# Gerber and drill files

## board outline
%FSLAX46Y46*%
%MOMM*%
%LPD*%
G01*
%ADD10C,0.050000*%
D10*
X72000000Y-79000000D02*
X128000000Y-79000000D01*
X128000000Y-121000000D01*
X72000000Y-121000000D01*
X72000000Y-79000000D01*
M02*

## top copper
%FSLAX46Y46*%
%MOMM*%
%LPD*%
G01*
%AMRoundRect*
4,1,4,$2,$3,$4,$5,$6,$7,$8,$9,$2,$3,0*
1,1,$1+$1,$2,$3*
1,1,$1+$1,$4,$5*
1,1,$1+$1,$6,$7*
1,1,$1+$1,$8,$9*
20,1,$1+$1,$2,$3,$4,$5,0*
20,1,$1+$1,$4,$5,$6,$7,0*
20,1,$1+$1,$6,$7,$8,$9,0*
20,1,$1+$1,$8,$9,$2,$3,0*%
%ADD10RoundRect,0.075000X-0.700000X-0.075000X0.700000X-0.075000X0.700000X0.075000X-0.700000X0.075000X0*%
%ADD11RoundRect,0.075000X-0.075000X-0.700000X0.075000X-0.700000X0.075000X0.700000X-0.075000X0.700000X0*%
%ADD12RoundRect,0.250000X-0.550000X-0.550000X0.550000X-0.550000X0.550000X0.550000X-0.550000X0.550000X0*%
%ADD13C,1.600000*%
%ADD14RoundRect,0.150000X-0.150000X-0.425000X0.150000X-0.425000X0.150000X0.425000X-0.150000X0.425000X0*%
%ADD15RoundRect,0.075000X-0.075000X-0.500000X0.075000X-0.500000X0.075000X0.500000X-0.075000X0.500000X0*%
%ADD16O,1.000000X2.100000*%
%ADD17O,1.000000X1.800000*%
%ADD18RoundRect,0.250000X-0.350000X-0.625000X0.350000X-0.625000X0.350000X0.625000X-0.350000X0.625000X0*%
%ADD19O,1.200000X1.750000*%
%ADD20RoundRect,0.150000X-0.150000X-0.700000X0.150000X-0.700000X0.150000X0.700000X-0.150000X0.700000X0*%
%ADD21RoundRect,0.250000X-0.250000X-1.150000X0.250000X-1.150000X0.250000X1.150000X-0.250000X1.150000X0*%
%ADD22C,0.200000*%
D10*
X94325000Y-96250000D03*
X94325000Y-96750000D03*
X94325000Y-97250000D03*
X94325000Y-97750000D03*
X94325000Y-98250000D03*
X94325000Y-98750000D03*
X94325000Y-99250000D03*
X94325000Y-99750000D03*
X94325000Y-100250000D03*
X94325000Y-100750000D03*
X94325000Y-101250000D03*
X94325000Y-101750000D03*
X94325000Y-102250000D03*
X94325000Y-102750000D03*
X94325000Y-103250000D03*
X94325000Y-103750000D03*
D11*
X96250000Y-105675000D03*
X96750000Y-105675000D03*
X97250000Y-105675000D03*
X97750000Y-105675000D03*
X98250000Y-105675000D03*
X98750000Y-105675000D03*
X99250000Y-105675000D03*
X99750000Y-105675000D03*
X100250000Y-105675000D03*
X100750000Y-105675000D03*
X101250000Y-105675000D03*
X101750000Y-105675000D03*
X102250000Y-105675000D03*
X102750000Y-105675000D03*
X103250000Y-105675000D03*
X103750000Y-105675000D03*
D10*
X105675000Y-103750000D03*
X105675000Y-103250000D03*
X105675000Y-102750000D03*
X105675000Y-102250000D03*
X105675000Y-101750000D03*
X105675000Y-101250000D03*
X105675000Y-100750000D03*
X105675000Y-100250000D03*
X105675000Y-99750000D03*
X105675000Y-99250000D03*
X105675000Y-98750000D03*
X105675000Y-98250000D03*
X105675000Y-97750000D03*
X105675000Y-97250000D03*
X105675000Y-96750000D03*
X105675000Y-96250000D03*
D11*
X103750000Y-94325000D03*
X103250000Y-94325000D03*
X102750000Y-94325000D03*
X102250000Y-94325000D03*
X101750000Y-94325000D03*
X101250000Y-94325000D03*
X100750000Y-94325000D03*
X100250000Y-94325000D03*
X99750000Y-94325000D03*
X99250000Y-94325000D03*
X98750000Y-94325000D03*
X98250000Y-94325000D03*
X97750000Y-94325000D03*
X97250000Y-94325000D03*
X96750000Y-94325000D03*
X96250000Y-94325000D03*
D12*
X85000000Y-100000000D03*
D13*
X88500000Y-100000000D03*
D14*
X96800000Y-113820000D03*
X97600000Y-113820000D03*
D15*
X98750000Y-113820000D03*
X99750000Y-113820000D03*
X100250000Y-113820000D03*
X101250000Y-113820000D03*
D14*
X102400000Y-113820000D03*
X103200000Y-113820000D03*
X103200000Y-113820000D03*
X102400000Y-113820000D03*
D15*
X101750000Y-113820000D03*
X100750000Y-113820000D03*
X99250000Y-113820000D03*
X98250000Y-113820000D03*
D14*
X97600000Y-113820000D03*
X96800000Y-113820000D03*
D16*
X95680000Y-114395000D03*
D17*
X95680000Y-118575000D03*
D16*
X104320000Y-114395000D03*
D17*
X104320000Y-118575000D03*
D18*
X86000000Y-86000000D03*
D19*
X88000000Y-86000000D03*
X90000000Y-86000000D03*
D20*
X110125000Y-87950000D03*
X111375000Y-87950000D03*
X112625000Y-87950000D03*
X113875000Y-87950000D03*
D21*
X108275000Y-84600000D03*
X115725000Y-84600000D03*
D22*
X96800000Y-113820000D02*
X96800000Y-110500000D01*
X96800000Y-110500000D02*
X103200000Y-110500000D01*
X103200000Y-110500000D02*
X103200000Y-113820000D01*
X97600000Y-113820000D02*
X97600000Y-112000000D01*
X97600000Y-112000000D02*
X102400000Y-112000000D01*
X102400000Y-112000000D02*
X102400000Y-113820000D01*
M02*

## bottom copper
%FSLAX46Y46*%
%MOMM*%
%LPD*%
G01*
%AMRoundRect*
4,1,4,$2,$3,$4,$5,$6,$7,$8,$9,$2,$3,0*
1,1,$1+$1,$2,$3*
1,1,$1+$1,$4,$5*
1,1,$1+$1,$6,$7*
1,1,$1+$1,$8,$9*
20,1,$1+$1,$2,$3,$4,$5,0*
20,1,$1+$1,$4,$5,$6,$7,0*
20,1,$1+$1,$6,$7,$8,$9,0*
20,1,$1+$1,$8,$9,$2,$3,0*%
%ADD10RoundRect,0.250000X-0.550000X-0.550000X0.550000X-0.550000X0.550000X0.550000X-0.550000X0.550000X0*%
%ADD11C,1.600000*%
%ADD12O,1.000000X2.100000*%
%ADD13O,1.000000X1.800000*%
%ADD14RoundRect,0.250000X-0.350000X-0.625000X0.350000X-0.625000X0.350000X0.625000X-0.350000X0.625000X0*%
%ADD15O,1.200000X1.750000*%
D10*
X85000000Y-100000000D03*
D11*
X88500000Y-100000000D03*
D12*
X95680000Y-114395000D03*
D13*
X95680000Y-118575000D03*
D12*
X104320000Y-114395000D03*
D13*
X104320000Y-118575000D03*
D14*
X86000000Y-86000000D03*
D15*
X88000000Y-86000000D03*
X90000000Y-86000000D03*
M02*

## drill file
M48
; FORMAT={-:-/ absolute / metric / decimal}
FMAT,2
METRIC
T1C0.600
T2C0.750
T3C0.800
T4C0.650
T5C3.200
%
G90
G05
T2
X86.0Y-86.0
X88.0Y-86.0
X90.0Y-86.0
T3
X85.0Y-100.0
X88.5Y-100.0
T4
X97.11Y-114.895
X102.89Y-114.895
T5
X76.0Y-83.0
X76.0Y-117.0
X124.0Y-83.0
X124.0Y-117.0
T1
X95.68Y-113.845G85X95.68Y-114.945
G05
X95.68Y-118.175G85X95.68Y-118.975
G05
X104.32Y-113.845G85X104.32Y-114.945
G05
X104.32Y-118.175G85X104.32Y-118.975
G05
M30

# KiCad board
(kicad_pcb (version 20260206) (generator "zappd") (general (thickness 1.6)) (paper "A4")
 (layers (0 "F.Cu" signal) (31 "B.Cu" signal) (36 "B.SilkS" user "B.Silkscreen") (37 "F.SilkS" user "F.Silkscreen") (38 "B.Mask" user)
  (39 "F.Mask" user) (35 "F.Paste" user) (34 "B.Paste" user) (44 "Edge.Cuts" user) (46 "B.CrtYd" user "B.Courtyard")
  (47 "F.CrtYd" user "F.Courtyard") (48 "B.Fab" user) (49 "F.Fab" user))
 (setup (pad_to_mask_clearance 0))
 (gr_rect (start 72.0 79.0) (end 128.0 121.0) (stroke (width 0.05) (type default)) (fill none) (layer "Edge.Cuts"))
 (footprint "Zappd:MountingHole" (layer "F.Cu") (at 76.0 83.0)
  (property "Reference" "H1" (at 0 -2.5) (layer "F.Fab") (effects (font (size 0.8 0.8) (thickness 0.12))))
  (pad "" np_thru_hole circle (at 0 0) (size 3.2 3.2) (drill 3.2) (layers "*.Cu" "*.Mask")))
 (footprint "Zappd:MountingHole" (layer "F.Cu") (at 124.0 83.0)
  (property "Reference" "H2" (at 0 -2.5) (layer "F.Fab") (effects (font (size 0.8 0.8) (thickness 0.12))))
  (pad "" np_thru_hole circle (at 0 0) (size 3.2 3.2) (drill 3.2) (layers "*.Cu" "*.Mask")))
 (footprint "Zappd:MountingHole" (layer "F.Cu") (at 124.0 117.0)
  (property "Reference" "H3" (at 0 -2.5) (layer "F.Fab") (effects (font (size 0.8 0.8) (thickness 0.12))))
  (pad "" np_thru_hole circle (at 0 0) (size 3.2 3.2) (drill 3.2) (layers "*.Cu" "*.Mask")))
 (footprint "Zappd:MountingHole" (layer "F.Cu") (at 76.0 117.0)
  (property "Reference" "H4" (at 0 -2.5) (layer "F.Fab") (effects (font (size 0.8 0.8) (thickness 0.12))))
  (pad "" np_thru_hole circle (at 0 0) (size 3.2 3.2) (drill 3.2) (layers "*.Cu" "*.Mask")))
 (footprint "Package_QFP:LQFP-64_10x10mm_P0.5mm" (layer "F.Cu") (at 100 100)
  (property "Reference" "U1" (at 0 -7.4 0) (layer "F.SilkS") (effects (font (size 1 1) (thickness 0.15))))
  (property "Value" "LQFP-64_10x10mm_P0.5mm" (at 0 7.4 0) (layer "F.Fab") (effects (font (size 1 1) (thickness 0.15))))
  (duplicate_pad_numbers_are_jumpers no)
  (pad "1" smd roundrect (at -5.675 -3.75) (size 1.55 0.3) (layers "F.Cu" "F.Mask" "F.Paste") (roundrect_rratio 0.25))
  (pad "2" smd roundrect (at -5.675 -3.25) (size 1.55 0.3) (layers "F.Cu" "F.Mask" "F.Paste") (roundrect_rratio 0.25))
  (pad "3" smd roundrect (at -5.675 -2.75) (size 1.55 0.3) (layers "F.Cu" "F.Mask" "F.Paste") (roundrect_rratio 0.25))
  (pad "4" smd roundrect (at -5.675 -2.25) (size 1.55 0.3) (layers "F.Cu" "F.Mask" "F.Paste") (roundrect_rratio 0.25))
  (pad "5" smd roundrect (at -5.675 -1.75) (size 1.55 0.3) (layers "F.Cu" "F.Mask" "F.Paste") (roundrect_rratio 0.25))
  (pad "6" smd roundrect (at -5.675 -1.25) (size 1.55 0.3) (layers "F.Cu" "F.Mask" "F.Paste") (roundrect_rratio 0.25))
  (pad "7" smd roundrect (at -5.675 -0.75) (size 1.55 0.3) (layers "F.Cu" "F.Mask" "F.Paste") (roundrect_rratio 0.25))
  (pad "8" smd roundrect (at -5.675 -0.25) (size 1.55 0.3) (layers "F.Cu" "F.Mask" "F.Paste") (roundrect_rratio 0.25))
  (pad "9" smd roundrect (at -5.675 0.25) (size 1.55 0.3) (layers "F.Cu" "F.Mask" "F.Paste") (roundrect_rratio 0.25))
  (pad "10" smd roundrect (at -5.675 0.75) (size 1.55 0.3) (layers "F.Cu" "F.Mask" "F.Paste") (roundrect_rratio 0.25))
  (pad "11" smd roundrect (at -5.675 1.25) (size 1.55 0.3) (layers "F.Cu" "F.Mask" "F.Paste") (roundrect_rratio 0.25))
  (pad "12" smd roundrect (at -5.675 1.75) (size 1.55 0.3) (layers "F.Cu" "F.Mask" "F.Paste") (roundrect_rratio 0.25))
  (pad "13" smd roundrect (at -5.675 2.25) (size 1.55 0.3) (layers "F.Cu" "F.Mask" "F.Paste") (roundrect_rratio 0.25))
  (pad "14" smd roundrect (at -5.675 2.75) (size 1.55 0.3) (layers "F.Cu" "F.Mask" "F.Paste") (roundrect_rratio 0.25))
  (pad "15" smd roundrect (at -5.675 3.25) (size 1.55 0.3) (layers "F.Cu" "F.Mask" "F.Paste") (roundrect_rratio 0.25))
  (pad "16" smd roundrect (at -5.675 3.75) (size 1.55 0.3) (layers "F.Cu" "F.Mask" "F.Paste") (roundrect_rratio 0.25))
  (pad "17" smd roundrect (at -3.75 5.675) (size 0.3 1.55) (layers "F.Cu" "F.Mask" "F.Paste") (roundrect_rratio 0.25))
  (pad "18" smd roundrect (at -3.25 5.675) (size 0.3 1.55) (layers "F.Cu" "F.Mask" "F.Paste") (roundrect_rratio 0.25))
  (pad "19" smd roundrect (at -2.75 5.675) (size 0.3 1.55) (layers "F.Cu" "F.Mask" "F.Paste") (roundrect_rratio 0.25))
  (pad "20" smd roundrect (at -2.25 5.675) (size 0.3 1.55) (layers "F.Cu" "F.Mask" "F.Paste") (roundrect_rratio 0.25))
  (pad "21" smd roundrect (at -1.75 5.675) (size 0.3 1.55) (layers "F.Cu" "F.Mask" "F.Paste") (roundrect_rratio 0.25))
  (pad "22" smd roundrect (at -1.25 5.675) (size 0.3 1.55) (layers "F.Cu" "F.Mask" "F.Paste") (roundrect_rratio 0.25))
  (pad "23" smd roundrect (at -0.75 5.675) (size 0.3 1.55) (layers "F.Cu" "F.Mask" "F.Paste") (roundrect_rratio 0.25))
  (pad "24" smd roundrect (at -0.25 5.675) (size 0.3 1.55) (layers "F.Cu" "F.Mask" "F.Paste") (roundrect_rratio 0.25))
  (pad "25" smd roundrect (at 0.25 5.675) (size 0.3 1.55) (layers "F.Cu" "F.Mask" "F.Paste") (roundrect_rratio 0.25))
  (pad "26" smd roundrect (at 0.75 5.675) (size 0.3 1.55) (layers "F.Cu" "F.Mask" "F.Paste") (roundrect_rratio 0.25))
  (pad "27" smd roundrect (at 1.25 5.675) (size 0.3 1.55) (layers "F.Cu" "F.Mask" "F.Paste") (roundrect_rratio 0.25))
  (pad "28" smd roundrect (at 1.75 5.675) (size 0.3 1.55) (layers "F.Cu" "F.Mask" "F.Paste") (roundrect_rratio 0.25))
  (pad "29" smd roundrect (at 2.25 5.675) (size 0.3 1.55) (layers "F.Cu" "F.Mask" "F.Paste") (roundrect_rratio 0.25))
  (pad "30" smd roundrect (at 2.75 5.675) (size 0.3 1.55) (layers "F.Cu" "F.Mask" "F.Paste") (roundrect_rratio 0.25))
  (pad "31" smd roundrect (at 3.25 5.675) (size 0.3 1.55) (layers "F.Cu" "F.Mask" "F.Paste") (roundrect_rratio 0.25))
  (pad "32" smd roundrect (at 3.75 5.675) (size 0.3 1.55) (layers "F.Cu" "F.Mask" "F.Paste") (roundrect_rratio 0.25))
  (pad "33" smd roundrect (at 5.675 3.75) (size 1.55 0.3) (layers "F.Cu" "F.Mask" "F.Paste") (roundrect_rratio 0.25))
  (pad "34" smd roundrect (at 5.675 3.25) (size 1.55 0.3) (layers "F.Cu" "F.Mask" "F.Paste") (roundrect_rratio 0.25))
  (pad "35" smd roundrect (at 5.675 2.75) (size 1.55 0.3) (layers "F.Cu" "F.Mask" "F.Paste") (roundrect_rratio 0.25))
  (pad "36" smd roundrect (at 5.675 2.25) (size 1.55 0.3) (layers "F.Cu" "F.Mask" "F.Paste") (roundrect_rratio 0.25))
  (pad "37" smd roundrect (at 5.675 1.75) (size 1.55 0.3) (layers "F.Cu" "F.Mask" "F.Paste") (roundrect_rratio 0.25))
  (pad "38" smd roundrect (at 5.675 1.25) (size 1.55 0.3) (layers "F.Cu" "F.Mask" "F.Paste") (roundrect_rratio 0.25))
  (pad "39" smd roundrect (at 5.675 0.75) (size 1.55 0.3) (layers "F.Cu" "F.Mask" "F.Paste") (roundrect_rratio 0.25))
  (pad "40" smd roundrect (at 5.675 0.25) (size 1.55 0.3) (layers "F.Cu" "F.Mask" "F.Paste") (roundrect_rratio 0.25))
  (pad "41" smd roundrect (at 5.675 -0.25) (size 1.55 0.3) (layers "F.Cu" "F.Mask" "F.Paste") (roundrect_rratio 0.25))
  (pad "42" smd roundrect (at 5.675 -0.75) (size 1.55 0.3) (layers "F.Cu" "F.Mask" "F.Paste") (roundrect_rratio 0.25))
  (pad "43" smd roundrect (at 5.675 -1.25) (size 1.55 0.3) (layers "F.Cu" "F.Mask" "F.Paste") (roundrect_rratio 0.25))
  (pad "44" smd roundrect (at 5.675 -1.75) (size 1.55 0.3) (layers "F.Cu" "F.Mask" "F.Paste") (roundrect_rratio 0.25))
  (pad "45" smd roundrect (at 5.675 -2.25) (size 1.55 0.3) (layers "F.Cu" "F.Mask" "F.Paste") (roundrect_rratio 0.25))
  (pad "46" smd roundrect (at 5.675 -2.75) (size 1.55 0.3) (layers "F.Cu" "F.Mask" "F.Paste") (roundrect_rratio 0.25))
  (pad "47" smd roundrect (at 5.675 -3.25) (size 1.55 0.3) (layers "F.Cu" "F.Mask" "F.Paste") (roundrect_rratio 0.25))
  (pad "48" smd roundrect (at 5.675 -3.75) (size 1.55 0.3) (layers "F.Cu" "F.Mask" "F.Paste") (roundrect_rratio 0.25))
  (pad "49" smd roundrect (at 3.75 -5.675) (size 0.3 1.55) (layers "F.Cu" "F.Mask" "F.Paste") (roundrect_rratio 0.25))
  (pad "50" smd roundrect (at 3.25 -5.675) (size 0.3 1.55) (layers "F.Cu" "F.Mask" "F.Paste") (roundrect_rratio 0.25))
  (pad "51" smd roundrect (at 2.75 -5.675) (size 0.3 1.55) (layers "F.Cu" "F.Mask" "F.Paste") (roundrect_rratio 0.25))
  (pad "52" smd roundrect (at 2.25 -5.675) (size 0.3 1.55) (layers "F.Cu" "F.Mask" "F.Paste") (roundrect_rratio 0.25))
  (pad "53" smd roundrect (at 1.75 -5.675) (size 0.3 1.55) (layers "F.Cu" "F.Mask" "F.Paste") (roundrect_rratio 0.25))
  (pad "54" smd roundrect (at 1.25 -5.675) (size 0.3 1.55) (layers "F.Cu" "F.Mask" "F.Paste") (roundrect_rratio 0.25))
  (pad "55" smd roundrect (at 0.75 -5.675) (size 0.3 1.55) (layers "F.Cu" "F.Mask" "F.Paste") (roundrect_rratio 0.25))
  (pad "56" smd roundrect (at 0.25 -5.675) (size 0.3 1.55) (layers "F.Cu" "F.Mask" "F.Paste") (roundrect_rratio 0.25))
  (pad "57" smd roundrect (at -0.25 -5.675) (size 0.3 1.55) (layers "F.Cu" "F.Mask" "F.Paste") (roundrect_rratio 0.25))
  (pad "58" smd roundrect (at -0.75 -5.675) (size 0.3 1.55) (layers "F.Cu" "F.Mask" "F.Paste") (roundrect_rratio 0.25))
  (pad "59" smd roundrect (at -1.25 -5.675) (size 0.3 1.55) (layers "F.Cu" "F.Mask" "F.Paste") (roundrect_rratio 0.25))
  (pad "60" smd roundrect (at -1.75 -5.675) (size 0.3 1.55) (layers "F.Cu" "F.Mask" "F.Paste") (roundrect_rratio 0.25))
  (pad "61" smd roundrect (at -2.25 -5.675) (size 0.3 1.55) (layers "F.Cu" "F.Mask" "F.Paste") (roundrect_rratio 0.25))
  (pad "62" smd roundrect (at -2.75 -5.675) (size 0.3 1.55) (layers "F.Cu" "F.Mask" "F.Paste") (roundrect_rratio 0.25))
  (pad "63" smd roundrect (at -3.25 -5.675) (size 0.3 1.55) (layers "F.Cu" "F.Mask" "F.Paste") (roundrect_rratio 0.25))
  (pad "64" smd roundrect (at -3.75 -5.675) (size 0.3 1.55) (layers "F.Cu" "F.Mask" "F.Paste") (roundrect_rratio 0.25)))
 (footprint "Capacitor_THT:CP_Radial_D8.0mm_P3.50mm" (layer "F.Cu") (at 85 100)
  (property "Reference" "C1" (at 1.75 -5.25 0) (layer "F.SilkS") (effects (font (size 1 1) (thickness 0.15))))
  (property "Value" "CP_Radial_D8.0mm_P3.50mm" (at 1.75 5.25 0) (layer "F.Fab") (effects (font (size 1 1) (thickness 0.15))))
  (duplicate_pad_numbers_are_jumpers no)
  (pad "1" thru_hole roundrect (at 0 0) (size 1.6 1.6) (drill 0.8) (layers "*.Cu" "*.Mask") (remove_unused_layers no)
   (roundrect_rratio 0.15625))
  (pad "2" thru_hole circle (at 3.5 0) (size 1.6 1.6) (drill 0.8) (layers "*.Cu" "*.Mask") (remove_unused_layers no)))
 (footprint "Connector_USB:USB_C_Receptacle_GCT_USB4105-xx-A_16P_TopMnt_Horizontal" (layer "F.Cu") (at 100 117.5)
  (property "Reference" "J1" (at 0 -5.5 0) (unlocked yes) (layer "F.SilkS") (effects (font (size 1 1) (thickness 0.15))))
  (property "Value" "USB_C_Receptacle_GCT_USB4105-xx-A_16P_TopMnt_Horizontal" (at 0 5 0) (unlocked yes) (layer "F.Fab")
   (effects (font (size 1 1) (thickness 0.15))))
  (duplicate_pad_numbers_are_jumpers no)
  (pad "" np_thru_hole circle (at -2.89 -2.605) (size 0.65 0.65) (drill 0.65) (layers "*.Cu" "*.Mask"))
  (pad "" np_thru_hole circle (at 2.89 -2.605) (size 0.65 0.65) (drill 0.65) (layers "*.Cu" "*.Mask"))
  (pad "A1" smd roundrect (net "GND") (at -3.2 -3.68) (size 0.6 1.15) (layers "F.Cu" "F.Mask" "F.Paste") (roundrect_rratio 0.25))
  (pad "A4" smd roundrect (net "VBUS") (at -2.4 -3.68) (size 0.6 1.15) (layers "F.Cu" "F.Mask" "F.Paste") (roundrect_rratio 0.25))
  (pad "A5" smd roundrect (at -1.25 -3.68) (size 0.3 1.15) (layers "F.Cu" "F.Mask" "F.Paste") (roundrect_rratio 0.25))
  (pad "A6" smd roundrect (at -0.25 -3.68) (size 0.3 1.15) (layers "F.Cu" "F.Mask" "F.Paste") (roundrect_rratio 0.25))
  (pad "A7" smd roundrect (at 0.25 -3.68) (size 0.3 1.15) (layers "F.Cu" "F.Mask" "F.Paste") (roundrect_rratio 0.25))
  (pad "A8" smd roundrect (at 1.25 -3.68) (size 0.3 1.15) (layers "F.Cu" "F.Mask" "F.Paste") (roundrect_rratio 0.25))
  (pad "A9" smd roundrect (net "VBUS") (at 2.4 -3.68) (size 0.6 1.15) (layers "F.Cu" "F.Mask" "F.Paste") (roundrect_rratio 0.25))
  (pad "A12" smd roundrect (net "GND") (at 3.2 -3.68) (size 0.6 1.15) (layers "F.Cu" "F.Mask" "F.Paste") (roundrect_rratio 0.25))
  (pad "B1" smd roundrect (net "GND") (at 3.2 -3.68) (size 0.6 1.15) (layers "F.Cu" "F.Mask" "F.Paste") (roundrect_rratio 0.25))
  (pad "B4" smd roundrect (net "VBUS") (at 2.4 -3.68) (size 0.6 1.15) (layers "F.Cu" "F.Mask" "F.Paste") (roundrect_rratio 0.25))
  (pad "B5" smd roundrect (at 1.75 -3.68) (size 0.3 1.15) (layers "F.Cu" "F.Mask" "F.Paste") (roundrect_rratio 0.25))
  (pad "B6" smd roundrect (at 0.75 -3.68) (size 0.3 1.15) (layers "F.Cu" "F.Mask" "F.Paste") (roundrect_rratio 0.25))
  (pad "B7" smd roundrect (at -0.75 -3.68) (size 0.3 1.15) (layers "F.Cu" "F.Mask" "F.Paste") (roundrect_rratio 0.25))
  (pad "B8" smd roundrect (at -1.75 -3.68) (size 0.3 1.15) (layers "F.Cu" "F.Mask" "F.Paste") (roundrect_rratio 0.25))
  (pad "B9" smd roundrect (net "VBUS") (at -2.4 -3.68) (size 0.6 1.15) (layers "F.Cu" "F.Mask" "F.Paste") (roundrect_rratio 0.25))
  (pad "B12" smd roundrect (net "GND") (at -3.2 -3.68) (size 0.6 1.15) (layers "F.Cu" "F.Mask" "F.Paste") (roundrect_rratio 0.25))
  (pad "SH" thru_hole oval (at -4.32 -3.105) (size 1 2.1) (drill oval 0.6 1.7) (layers "*.Cu" "*.Mask" "F.Paste") (remove_unused_layers no))
  (pad "SH" thru_hole oval (at -4.32 1.075) (size 1 1.8) (drill oval 0.6 1.4) (layers "*.Cu" "*.Mask" "F.Paste") (remove_unused_layers no))
  (pad "SH" thru_hole oval (at 4.32 -3.105) (size 1 2.1) (drill oval 0.6 1.7) (layers "*.Cu" "*.Mask" "F.Paste") (remove_unused_layers no))
  (pad "SH" thru_hole oval (at 4.32 1.075) (size 1 1.8) (drill oval 0.6 1.4) (layers "*.Cu" "*.Mask" "F.Paste") (remove_unused_layers no)))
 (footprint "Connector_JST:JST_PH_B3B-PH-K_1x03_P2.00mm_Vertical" (layer "F.Cu") (at 86 86)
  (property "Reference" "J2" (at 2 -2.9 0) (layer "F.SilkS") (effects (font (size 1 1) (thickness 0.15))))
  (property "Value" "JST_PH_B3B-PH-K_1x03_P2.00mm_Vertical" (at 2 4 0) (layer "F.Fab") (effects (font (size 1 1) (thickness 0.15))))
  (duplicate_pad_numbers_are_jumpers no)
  (pad "1" thru_hole roundrect (at 0 0) (size 1.2 1.75) (drill 0.75) (layers "*.Cu" "*.Mask") (remove_unused_layers no)
   (roundrect_rratio 0.208333))
  (pad "2" thru_hole oval (at 2 0) (size 1.2 1.75) (drill 0.75) (layers "*.Cu" "*.Mask") (remove_unused_layers no))
  (pad "3" thru_hole oval (at 4 0) (size 1.2 1.75) (drill 0.75) (layers "*.Cu" "*.Mask") (remove_unused_layers no)))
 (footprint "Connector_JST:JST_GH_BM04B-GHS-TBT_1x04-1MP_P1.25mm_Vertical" (layer "F.Cu") (at 112 86)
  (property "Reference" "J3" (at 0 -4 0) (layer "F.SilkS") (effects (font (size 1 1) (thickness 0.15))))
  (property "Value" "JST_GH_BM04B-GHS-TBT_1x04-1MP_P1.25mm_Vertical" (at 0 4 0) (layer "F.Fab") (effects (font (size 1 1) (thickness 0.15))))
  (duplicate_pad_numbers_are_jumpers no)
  (pad "1" smd roundrect (at -1.875 1.95) (size 0.6 1.7) (layers "F.Cu" "F.Mask" "F.Paste") (roundrect_rratio 0.25))
  (pad "2" smd roundrect (at -0.625 1.95) (size 0.6 1.7) (layers "F.Cu" "F.Mask" "F.Paste") (roundrect_rratio 0.25))
  (pad "3" smd roundrect (at 0.625 1.95) (size 0.6 1.7) (layers "F.Cu" "F.Mask" "F.Paste") (roundrect_rratio 0.25))
  (pad "4" smd roundrect (at 1.875 1.95) (size 0.6 1.7) (layers "F.Cu" "F.Mask" "F.Paste") (roundrect_rratio 0.25))
  (pad "MP" smd roundrect (at -3.725 -1.4) (size 1 2.8) (layers "F.Cu" "F.Mask" "F.Paste") (roundrect_rratio 0.25))
  (pad "MP" smd roundrect (at 3.725 -1.4) (size 1 2.8) (layers "F.Cu" "F.Mask" "F.Paste") (roundrect_rratio 0.25)))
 (segment (start 96.8000 113.8200) (end 96.8000 110.5000) (width 0.2) (layer "F.Cu") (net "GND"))
 (segment (start 96.8000 110.5000) (end 103.2000 110.5000) (width 0.2) (layer "F.Cu") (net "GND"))
 (segment (start 103.2000 110.5000) (end 103.2000 113.8200) (width 0.2) (layer "F.Cu") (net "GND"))
 (segment (start 97.6000 113.8200) (end 97.6000 112.0000) (width 0.2) (layer "F.Cu") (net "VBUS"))
 (segment (start 97.6000 112.0000) (end 102.4000 112.0000) (width 0.2) (layer "F.Cu") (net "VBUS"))
 (segment (start 102.4000 112.0000) (end 102.4000 113.8200) (width 0.2) (layer "F.Cu") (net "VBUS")))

